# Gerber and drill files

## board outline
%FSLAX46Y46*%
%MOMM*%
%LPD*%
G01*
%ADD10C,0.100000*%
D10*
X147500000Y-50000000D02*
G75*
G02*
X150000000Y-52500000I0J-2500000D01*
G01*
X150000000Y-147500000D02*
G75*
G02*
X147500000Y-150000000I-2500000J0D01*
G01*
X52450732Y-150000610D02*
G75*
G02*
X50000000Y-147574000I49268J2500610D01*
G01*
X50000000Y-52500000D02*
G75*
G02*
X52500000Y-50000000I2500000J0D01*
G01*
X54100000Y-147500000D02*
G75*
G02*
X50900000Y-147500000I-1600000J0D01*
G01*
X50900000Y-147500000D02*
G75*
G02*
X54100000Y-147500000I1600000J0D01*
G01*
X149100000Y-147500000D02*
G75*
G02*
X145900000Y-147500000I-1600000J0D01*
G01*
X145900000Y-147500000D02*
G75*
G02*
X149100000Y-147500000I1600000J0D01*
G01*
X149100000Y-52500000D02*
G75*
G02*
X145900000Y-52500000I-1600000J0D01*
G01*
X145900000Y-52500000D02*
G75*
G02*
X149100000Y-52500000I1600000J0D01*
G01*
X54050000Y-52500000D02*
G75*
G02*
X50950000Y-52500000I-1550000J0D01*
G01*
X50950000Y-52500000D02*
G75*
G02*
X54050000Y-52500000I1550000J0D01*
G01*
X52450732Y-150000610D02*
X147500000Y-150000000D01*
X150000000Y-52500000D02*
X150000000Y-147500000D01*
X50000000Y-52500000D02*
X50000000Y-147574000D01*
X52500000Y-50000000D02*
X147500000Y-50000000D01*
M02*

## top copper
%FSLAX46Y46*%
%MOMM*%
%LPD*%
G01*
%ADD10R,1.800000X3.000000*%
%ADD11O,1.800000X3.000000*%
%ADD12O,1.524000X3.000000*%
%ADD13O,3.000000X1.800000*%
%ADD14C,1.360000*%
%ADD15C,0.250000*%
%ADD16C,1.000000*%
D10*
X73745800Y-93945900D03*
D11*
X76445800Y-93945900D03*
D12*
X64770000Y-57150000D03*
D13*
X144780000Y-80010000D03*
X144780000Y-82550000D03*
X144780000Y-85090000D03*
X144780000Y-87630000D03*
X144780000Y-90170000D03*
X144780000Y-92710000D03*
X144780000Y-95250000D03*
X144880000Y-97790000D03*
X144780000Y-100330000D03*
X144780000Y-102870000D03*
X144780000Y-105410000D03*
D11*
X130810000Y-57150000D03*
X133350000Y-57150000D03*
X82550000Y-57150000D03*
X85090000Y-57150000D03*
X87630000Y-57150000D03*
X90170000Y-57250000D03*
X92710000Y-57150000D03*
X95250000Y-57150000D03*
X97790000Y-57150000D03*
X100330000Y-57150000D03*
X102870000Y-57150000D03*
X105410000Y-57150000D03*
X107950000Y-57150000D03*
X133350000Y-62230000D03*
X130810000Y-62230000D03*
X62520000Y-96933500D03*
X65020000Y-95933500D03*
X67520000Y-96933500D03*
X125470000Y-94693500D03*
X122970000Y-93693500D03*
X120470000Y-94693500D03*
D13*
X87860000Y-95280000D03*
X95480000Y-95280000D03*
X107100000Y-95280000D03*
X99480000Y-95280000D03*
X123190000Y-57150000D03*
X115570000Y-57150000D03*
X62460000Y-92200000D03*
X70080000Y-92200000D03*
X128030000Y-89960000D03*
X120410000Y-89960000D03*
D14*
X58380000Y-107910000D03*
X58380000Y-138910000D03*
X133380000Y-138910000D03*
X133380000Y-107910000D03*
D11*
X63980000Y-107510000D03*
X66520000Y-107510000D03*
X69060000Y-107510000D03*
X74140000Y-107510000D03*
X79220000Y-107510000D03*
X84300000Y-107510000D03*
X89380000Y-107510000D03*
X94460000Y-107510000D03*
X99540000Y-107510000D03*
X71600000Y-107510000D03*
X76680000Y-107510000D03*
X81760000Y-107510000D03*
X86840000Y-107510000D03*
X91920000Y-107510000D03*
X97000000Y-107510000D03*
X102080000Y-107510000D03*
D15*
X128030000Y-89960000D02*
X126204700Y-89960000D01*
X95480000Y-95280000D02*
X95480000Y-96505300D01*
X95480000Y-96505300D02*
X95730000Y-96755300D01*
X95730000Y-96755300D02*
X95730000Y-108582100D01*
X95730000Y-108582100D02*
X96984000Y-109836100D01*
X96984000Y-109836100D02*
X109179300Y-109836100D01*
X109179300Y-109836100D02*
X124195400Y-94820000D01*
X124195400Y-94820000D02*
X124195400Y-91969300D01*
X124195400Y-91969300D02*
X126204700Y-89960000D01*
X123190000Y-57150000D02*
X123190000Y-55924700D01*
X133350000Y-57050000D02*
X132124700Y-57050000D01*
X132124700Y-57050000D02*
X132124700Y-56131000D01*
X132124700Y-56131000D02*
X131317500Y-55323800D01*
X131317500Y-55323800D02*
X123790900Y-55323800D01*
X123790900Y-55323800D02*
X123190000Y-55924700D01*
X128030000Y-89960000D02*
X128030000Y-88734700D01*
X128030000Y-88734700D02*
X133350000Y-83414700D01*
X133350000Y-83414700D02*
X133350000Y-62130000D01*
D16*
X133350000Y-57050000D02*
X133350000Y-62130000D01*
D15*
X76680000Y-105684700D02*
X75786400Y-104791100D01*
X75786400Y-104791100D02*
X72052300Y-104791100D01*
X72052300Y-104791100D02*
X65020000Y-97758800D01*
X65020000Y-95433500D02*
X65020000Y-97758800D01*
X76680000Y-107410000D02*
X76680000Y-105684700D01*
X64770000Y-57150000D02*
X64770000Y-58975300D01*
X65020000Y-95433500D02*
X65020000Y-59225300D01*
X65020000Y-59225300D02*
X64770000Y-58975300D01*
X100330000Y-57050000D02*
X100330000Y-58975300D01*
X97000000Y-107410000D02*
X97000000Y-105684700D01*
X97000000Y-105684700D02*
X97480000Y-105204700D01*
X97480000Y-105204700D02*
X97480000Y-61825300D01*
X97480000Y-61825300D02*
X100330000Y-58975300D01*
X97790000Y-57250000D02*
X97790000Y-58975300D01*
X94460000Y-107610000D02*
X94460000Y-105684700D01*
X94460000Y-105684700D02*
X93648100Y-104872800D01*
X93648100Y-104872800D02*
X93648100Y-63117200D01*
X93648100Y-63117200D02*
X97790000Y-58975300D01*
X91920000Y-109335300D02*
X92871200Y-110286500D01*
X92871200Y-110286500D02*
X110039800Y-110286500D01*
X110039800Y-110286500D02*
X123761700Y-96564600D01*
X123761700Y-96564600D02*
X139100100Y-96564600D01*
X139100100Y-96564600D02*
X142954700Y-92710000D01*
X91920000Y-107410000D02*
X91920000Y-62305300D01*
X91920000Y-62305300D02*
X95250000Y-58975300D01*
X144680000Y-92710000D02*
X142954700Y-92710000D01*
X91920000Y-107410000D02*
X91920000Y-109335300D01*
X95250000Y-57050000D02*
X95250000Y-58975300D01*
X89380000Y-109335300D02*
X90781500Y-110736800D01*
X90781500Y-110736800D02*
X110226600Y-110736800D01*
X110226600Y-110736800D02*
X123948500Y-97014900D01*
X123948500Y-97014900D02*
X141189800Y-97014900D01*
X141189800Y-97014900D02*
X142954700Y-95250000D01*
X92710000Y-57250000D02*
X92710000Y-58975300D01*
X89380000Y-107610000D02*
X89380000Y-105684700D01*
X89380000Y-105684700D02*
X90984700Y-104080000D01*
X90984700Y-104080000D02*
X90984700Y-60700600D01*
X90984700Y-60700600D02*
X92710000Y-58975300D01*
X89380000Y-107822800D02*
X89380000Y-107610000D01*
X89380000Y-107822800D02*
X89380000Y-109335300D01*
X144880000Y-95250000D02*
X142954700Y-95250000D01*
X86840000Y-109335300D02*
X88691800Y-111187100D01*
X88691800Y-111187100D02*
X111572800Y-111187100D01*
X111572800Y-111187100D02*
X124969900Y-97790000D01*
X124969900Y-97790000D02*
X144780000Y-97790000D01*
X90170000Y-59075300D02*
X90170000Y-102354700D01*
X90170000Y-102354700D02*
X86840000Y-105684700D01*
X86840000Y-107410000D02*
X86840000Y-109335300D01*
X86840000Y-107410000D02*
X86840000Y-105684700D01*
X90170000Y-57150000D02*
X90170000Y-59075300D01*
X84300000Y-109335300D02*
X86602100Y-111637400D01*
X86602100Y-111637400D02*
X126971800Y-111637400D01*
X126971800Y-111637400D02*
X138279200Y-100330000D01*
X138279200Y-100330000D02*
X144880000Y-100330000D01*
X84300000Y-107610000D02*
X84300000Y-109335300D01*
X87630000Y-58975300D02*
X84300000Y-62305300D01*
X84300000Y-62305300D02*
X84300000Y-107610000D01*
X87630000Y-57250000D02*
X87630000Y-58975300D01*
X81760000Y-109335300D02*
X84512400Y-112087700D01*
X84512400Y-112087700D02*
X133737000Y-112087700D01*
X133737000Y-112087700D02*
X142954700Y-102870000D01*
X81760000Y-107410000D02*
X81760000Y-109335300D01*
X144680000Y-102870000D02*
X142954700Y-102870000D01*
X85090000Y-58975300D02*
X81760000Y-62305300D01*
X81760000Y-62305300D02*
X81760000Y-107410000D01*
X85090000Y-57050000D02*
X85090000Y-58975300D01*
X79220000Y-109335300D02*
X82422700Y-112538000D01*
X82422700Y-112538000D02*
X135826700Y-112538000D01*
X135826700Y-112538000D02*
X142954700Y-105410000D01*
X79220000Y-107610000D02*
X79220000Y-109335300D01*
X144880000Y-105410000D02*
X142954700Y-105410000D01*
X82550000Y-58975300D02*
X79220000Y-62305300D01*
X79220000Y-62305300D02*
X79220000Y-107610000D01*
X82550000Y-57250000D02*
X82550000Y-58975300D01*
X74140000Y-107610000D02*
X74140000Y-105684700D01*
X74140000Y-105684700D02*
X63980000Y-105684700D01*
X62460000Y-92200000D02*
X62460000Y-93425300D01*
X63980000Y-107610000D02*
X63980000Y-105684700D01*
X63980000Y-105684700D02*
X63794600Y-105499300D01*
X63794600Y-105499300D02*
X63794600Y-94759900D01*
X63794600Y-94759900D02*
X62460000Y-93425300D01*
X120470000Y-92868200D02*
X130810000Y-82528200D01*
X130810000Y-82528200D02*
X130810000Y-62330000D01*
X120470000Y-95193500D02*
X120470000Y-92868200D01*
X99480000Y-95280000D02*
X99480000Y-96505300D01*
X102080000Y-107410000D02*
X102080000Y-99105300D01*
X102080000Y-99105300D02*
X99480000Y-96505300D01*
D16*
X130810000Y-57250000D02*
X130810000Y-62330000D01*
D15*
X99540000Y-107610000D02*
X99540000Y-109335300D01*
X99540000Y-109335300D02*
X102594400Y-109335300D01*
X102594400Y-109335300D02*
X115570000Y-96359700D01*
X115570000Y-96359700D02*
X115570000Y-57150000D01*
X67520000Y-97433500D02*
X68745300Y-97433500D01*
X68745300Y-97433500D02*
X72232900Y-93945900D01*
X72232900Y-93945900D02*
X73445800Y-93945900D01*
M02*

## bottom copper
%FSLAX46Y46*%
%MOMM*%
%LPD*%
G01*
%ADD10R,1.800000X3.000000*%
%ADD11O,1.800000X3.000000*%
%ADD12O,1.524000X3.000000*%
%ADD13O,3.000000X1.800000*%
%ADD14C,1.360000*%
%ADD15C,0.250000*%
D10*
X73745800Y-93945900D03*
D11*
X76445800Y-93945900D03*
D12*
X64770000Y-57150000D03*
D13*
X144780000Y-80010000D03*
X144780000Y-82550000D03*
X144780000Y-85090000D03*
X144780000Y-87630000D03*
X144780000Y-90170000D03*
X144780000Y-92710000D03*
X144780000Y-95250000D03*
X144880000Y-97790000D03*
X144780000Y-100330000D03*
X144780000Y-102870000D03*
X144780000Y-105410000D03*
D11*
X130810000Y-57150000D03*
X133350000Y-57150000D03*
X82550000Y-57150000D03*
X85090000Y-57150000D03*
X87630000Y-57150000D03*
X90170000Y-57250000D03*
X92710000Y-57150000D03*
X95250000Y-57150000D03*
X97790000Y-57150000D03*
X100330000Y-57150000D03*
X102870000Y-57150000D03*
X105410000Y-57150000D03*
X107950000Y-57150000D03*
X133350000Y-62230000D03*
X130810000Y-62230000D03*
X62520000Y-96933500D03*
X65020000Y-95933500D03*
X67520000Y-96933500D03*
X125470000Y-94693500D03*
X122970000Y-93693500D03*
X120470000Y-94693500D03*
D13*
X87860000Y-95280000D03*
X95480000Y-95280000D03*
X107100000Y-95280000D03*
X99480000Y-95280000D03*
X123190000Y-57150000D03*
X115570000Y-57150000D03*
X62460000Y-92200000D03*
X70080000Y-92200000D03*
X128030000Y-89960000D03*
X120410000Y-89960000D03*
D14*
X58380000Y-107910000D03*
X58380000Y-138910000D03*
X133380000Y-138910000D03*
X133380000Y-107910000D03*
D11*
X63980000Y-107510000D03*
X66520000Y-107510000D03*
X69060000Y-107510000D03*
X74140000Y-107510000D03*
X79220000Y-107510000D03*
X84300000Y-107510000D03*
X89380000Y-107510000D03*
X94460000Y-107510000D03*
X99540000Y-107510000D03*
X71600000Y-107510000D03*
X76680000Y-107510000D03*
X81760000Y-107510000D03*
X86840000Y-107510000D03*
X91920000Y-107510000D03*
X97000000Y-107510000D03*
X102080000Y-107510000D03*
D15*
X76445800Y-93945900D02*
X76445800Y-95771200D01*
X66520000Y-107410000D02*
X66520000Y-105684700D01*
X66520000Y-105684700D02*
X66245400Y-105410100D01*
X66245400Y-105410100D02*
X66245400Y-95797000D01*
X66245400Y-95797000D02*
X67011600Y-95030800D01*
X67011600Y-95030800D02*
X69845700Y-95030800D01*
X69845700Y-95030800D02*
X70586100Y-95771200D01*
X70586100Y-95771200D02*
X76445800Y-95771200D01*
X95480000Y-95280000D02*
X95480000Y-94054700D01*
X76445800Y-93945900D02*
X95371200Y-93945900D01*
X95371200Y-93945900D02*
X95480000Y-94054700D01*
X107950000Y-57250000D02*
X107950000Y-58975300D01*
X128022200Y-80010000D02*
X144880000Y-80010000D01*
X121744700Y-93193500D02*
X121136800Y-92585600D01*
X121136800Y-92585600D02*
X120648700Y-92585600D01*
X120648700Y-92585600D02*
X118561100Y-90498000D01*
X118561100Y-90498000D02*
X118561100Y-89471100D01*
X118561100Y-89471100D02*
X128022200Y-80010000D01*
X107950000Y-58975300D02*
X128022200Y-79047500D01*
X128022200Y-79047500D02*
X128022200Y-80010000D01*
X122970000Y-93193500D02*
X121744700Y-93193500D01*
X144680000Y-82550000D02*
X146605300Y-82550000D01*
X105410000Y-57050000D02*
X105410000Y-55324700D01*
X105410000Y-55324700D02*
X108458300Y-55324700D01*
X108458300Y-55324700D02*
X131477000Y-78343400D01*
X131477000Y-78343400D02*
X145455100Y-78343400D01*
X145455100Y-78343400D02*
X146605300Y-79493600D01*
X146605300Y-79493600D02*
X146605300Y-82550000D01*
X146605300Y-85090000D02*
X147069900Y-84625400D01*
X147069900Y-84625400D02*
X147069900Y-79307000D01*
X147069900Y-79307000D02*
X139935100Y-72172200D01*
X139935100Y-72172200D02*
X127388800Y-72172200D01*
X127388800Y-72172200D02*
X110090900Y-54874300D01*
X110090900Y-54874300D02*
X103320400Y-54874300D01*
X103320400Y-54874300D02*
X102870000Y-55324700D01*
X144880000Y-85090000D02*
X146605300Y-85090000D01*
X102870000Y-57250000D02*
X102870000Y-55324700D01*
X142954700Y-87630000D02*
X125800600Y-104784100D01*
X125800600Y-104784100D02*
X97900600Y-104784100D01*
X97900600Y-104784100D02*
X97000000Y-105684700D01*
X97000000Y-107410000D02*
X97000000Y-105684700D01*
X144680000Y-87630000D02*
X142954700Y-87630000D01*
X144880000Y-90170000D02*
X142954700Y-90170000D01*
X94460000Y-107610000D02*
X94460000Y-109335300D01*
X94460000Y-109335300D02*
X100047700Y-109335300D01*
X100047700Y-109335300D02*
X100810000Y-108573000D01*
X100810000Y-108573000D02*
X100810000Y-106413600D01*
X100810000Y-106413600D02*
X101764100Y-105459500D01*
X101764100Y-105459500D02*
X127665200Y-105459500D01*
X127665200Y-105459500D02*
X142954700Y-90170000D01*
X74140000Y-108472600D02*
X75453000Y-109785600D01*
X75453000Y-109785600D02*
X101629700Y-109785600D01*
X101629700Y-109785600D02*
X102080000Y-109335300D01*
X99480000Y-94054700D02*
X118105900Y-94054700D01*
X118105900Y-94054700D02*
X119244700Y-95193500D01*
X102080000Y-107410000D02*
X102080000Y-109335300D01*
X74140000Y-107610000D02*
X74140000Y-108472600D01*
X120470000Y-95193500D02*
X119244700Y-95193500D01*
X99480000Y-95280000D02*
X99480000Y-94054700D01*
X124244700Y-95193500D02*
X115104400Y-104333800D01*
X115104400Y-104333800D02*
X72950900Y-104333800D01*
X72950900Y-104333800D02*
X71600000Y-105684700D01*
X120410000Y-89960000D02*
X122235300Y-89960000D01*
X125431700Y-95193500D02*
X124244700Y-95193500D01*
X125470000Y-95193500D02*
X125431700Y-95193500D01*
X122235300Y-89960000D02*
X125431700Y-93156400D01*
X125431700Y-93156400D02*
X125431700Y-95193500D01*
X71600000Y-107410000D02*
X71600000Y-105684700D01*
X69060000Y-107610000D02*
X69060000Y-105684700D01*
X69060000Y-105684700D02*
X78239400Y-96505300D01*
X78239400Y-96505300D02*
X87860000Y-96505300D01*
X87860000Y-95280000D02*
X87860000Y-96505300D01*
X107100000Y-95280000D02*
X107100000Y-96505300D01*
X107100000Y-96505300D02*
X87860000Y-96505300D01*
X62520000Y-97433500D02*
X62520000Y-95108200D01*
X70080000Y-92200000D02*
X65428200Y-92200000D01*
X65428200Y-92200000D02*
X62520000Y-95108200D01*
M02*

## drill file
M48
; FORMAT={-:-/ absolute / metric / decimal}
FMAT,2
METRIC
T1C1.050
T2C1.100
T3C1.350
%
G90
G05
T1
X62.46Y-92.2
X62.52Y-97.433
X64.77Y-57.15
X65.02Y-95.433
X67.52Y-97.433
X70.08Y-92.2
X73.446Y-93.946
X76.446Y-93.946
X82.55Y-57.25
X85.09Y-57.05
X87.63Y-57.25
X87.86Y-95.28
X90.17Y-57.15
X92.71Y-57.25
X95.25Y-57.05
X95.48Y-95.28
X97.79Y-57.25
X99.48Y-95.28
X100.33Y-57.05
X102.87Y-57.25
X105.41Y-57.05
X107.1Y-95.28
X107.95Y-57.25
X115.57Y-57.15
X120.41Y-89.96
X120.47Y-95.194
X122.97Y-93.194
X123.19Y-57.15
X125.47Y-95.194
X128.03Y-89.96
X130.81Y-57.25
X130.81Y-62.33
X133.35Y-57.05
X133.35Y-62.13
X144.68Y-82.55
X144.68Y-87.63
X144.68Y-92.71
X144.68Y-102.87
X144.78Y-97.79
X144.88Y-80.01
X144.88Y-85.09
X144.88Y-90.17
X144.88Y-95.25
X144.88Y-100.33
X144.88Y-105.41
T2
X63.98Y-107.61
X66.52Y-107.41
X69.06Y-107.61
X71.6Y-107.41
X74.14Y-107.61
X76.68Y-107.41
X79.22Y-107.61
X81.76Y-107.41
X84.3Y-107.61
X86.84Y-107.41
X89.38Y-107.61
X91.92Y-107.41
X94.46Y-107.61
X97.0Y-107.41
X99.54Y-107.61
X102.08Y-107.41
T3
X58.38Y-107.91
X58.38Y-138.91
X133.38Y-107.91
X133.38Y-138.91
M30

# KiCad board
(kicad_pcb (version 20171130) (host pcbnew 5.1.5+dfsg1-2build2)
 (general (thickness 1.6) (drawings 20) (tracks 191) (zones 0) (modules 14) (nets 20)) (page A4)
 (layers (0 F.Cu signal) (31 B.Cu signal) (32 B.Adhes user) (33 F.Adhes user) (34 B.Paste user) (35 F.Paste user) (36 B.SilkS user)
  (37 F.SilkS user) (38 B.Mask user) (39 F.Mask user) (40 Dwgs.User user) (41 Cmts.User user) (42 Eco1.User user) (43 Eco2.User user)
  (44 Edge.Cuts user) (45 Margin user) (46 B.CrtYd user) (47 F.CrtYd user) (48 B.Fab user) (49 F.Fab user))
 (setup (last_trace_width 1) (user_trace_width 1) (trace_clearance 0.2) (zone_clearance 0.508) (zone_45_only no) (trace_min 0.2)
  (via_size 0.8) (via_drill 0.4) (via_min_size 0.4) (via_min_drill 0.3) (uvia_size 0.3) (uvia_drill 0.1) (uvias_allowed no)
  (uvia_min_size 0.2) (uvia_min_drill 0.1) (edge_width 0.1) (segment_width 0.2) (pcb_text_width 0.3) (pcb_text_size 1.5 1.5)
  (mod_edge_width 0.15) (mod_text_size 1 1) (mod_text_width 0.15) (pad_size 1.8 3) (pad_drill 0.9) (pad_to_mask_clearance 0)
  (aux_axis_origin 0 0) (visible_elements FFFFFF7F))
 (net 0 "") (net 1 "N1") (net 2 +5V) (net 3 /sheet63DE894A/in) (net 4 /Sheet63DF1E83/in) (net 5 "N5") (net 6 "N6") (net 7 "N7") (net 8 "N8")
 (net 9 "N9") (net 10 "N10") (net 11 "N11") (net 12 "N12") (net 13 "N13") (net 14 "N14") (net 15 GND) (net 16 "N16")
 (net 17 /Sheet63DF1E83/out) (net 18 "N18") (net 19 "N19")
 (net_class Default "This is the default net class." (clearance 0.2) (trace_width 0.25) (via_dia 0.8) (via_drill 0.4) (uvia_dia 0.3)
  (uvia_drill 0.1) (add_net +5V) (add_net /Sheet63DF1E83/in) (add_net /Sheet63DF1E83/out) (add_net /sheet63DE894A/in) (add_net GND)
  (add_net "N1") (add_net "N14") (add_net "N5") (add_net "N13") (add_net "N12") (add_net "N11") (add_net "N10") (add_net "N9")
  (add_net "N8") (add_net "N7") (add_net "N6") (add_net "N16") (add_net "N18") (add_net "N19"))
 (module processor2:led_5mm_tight (layer F.Cu) (at 74.9458 93.9459)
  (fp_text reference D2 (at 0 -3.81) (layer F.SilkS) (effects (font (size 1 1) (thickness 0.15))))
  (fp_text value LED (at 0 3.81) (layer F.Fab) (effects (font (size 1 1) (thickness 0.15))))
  (pad 1 thru_hole rect (at -1.5 0) (size 1.8 3) (drill 1.05 (offset 0.3 0)) (layers *.Cu *.Mask) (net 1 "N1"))
  (pad 2 thru_hole oval (at 1.5 0) (size 1.8 3) (drill 1.05) (layers *.Cu *.Mask) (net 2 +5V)))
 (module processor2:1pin (layer F.Cu) (at 64.77 57.15 90)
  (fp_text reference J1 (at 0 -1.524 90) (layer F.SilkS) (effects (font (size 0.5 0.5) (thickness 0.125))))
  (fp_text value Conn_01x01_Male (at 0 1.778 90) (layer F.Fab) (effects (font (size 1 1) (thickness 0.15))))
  (pad 1 thru_hole oval (at 0 0 90) (size 3 1.524) (drill 1.05) (layers *.Cu *.Mask) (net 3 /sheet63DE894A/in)))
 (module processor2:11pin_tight (layer F.Cu) (at 144.78 105.41 90)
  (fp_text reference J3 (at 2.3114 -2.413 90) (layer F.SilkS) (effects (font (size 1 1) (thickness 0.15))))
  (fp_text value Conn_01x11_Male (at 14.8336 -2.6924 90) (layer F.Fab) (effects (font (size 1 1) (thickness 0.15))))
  (pad 11 thru_hole oval (at 25.4 0.1 90) (size 1.8 3) (drill 1.05 (offset 0 -0.1)) (layers *.Cu *.Mask) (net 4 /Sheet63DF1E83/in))
  (pad 10 thru_hole oval (at 22.86 -0.1 90) (size 1.8 3) (drill 1.05 (offset 0 0.1)) (layers *.Cu *.Mask) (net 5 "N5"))
  (pad 9 thru_hole oval (at 20.32 0.1 90) (size 1.8 3) (drill 1.05 (offset 0 -0.1)) (layers *.Cu *.Mask) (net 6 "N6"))
  (pad 8 thru_hole oval (at 17.78 -0.1 90) (size 1.8 3) (drill 1.05 (offset 0 0.1)) (layers *.Cu *.Mask) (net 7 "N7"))
  (pad 7 thru_hole oval (at 15.24 0.1 90) (size 1.8 3) (drill 1.05 (offset 0 -0.1)) (layers *.Cu *.Mask) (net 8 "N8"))
  (pad 6 thru_hole oval (at 12.7 -0.1 90) (size 1.8 3) (drill 1.05 (offset 0 0.1)) (layers *.Cu *.Mask) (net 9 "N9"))
  (pad 5 thru_hole oval (at 10.16 0.1 90) (size 1.8 3) (drill 1.05 (offset 0 -0.1)) (layers *.Cu *.Mask) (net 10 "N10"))
  (pad 4 thru_hole oval (at 7.62 0 90) (size 1.8 3) (drill 1.05 (offset 0 0.1)) (layers *.Cu *.Mask) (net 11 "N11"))
  (pad 3 thru_hole oval (at 5.08 0.1 90) (size 1.8 3) (drill 1.05 (offset 0 -0.1)) (layers *.Cu *.Mask) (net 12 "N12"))
  (pad 2 thru_hole oval (at 2.54 -0.1 90) (size 1.8 3) (drill 1.05 (offset 0 0.1)) (layers *.Cu *.Mask) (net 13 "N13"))
  (pad 1 thru_hole oval (at 0 0.1 90) (size 1.8 3) (drill 1.05 (offset 0 -0.1)) (layers *.Cu *.Mask) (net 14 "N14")))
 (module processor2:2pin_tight (layer F.Cu) (at 133.35 57.15)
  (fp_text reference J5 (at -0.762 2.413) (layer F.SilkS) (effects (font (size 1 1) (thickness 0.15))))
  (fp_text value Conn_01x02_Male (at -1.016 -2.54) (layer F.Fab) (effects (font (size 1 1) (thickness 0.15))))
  (pad 2 thru_hole oval (at -2.54 0.1) (size 1.8 3) (drill 1.05 (offset 0 -0.1)) (layers *.Cu *.Mask) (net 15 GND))
  (pad 1 thru_hole oval (at 0 -0.1) (size 1.8 3) (drill 1.05 (offset 0 0.1)) (layers *.Cu *.Mask) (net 2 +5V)))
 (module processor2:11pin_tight (layer F.Cu) (at 82.55 57.15)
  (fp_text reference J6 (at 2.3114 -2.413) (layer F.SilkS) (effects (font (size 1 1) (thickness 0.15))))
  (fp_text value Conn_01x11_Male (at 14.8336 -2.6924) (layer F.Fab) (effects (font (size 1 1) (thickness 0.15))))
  (pad 1 thru_hole oval (at 0 0.1) (size 1.8 3) (drill 1.05 (offset 0 -0.1)) (layers *.Cu *.Mask) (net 14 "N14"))
  (pad 2 thru_hole oval (at 2.54 -0.1) (size 1.8 3) (drill 1.05 (offset 0 0.1)) (layers *.Cu *.Mask) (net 13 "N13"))
  (pad 3 thru_hole oval (at 5.08 0.1) (size 1.8 3) (drill 1.05 (offset 0 -0.1)) (layers *.Cu *.Mask) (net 12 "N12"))
  (pad 4 thru_hole oval (at 7.62 0) (size 1.8 3) (drill 1.05 (offset 0 0.1)) (layers *.Cu *.Mask) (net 11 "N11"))
  (pad 5 thru_hole oval (at 10.16 0.1) (size 1.8 3) (drill 1.05 (offset 0 -0.1)) (layers *.Cu *.Mask) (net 10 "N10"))
  (pad 6 thru_hole oval (at 12.7 -0.1) (size 1.8 3) (drill 1.05 (offset 0 0.1)) (layers *.Cu *.Mask) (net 9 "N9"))
  (pad 7 thru_hole oval (at 15.24 0.1) (size 1.8 3) (drill 1.05 (offset 0 -0.1)) (layers *.Cu *.Mask) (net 8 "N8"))
  (pad 8 thru_hole oval (at 17.78 -0.1) (size 1.8 3) (drill 1.05 (offset 0 0.1)) (layers *.Cu *.Mask) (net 7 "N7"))
  (pad 9 thru_hole oval (at 20.32 0.1) (size 1.8 3) (drill 1.05 (offset 0 -0.1)) (layers *.Cu *.Mask) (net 6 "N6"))
  (pad 10 thru_hole oval (at 22.86 -0.1) (size 1.8 3) (drill 1.05 (offset 0 0.1)) (layers *.Cu *.Mask) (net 5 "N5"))
  (pad 11 thru_hole oval (at 25.4 0.1) (size 1.8 3) (drill 1.05 (offset 0 -0.1)) (layers *.Cu *.Mask) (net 4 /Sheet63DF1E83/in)))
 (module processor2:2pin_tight (layer F.Cu) (at 133.35 62.23)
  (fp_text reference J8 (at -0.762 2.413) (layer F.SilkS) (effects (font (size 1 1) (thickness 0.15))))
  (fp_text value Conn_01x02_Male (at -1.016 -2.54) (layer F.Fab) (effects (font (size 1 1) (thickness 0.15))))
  (pad 1 thru_hole oval (at 0 -0.1) (size 1.8 3) (drill 1.05 (offset 0 0.1)) (layers *.Cu *.Mask) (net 2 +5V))
  (pad 2 thru_hole oval (at -2.54 0.1) (size 1.8 3) (drill 1.05 (offset 0 -0.1)) (layers *.Cu *.Mask) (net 15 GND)))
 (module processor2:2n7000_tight (layer F.Cu) (at 65.02 96.4335)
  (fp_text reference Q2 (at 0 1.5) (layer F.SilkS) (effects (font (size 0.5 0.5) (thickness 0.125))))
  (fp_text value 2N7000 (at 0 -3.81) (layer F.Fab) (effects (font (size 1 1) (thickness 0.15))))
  (pad 1 thru_hole oval (at -2.5 1) (size 1.8 3) (drill 1.05 (offset 0 -0.5)) (layers *.Cu *.Mask) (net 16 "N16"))
  (pad 2 thru_hole oval (at 0 -1) (size 1.8 3) (drill 1.05 (offset 0 0.5)) (layers *.Cu *.Mask) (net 3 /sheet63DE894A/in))
  (pad 3 thru_hole oval (at 2.5 1) (size 1.8 3) (drill 1.05 (offset 0 -0.5)) (layers *.Cu *.Mask) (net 1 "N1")))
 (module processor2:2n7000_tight (layer F.Cu) (at 122.97 94.1935)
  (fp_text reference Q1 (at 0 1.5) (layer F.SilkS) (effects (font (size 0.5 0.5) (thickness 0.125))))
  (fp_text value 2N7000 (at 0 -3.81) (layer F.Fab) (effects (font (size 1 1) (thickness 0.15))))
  (pad 3 thru_hole oval (at 2.5 1) (size 1.8 3) (drill 1.05 (offset 0 -0.5)) (layers *.Cu *.Mask) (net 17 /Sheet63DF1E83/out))
  (pad 2 thru_hole oval (at 0 -1) (size 1.8 3) (drill 1.05 (offset 0 0.5)) (layers *.Cu *.Mask) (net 4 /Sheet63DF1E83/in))
  (pad 1 thru_hole oval (at -2.5 1) (size 1.8 3) (drill 1.05 (offset 0 -0.5)) (layers *.Cu *.Mask) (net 15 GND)))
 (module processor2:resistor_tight (layer F.Cu) (at 91.67 95.28)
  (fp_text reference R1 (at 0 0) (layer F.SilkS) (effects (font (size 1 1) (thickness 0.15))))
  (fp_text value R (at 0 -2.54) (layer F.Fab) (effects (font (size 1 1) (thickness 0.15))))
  (pad 2 thru_hole oval (at -3.81 0 90) (size 1.8 3) (drill 1.05) (layers *.Cu *.Mask) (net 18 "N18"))
  (pad 1 thru_hole oval (at 3.81 0 90) (size 1.8 3) (drill 1.05) (layers *.Cu *.Mask) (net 2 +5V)))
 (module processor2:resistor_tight (layer F.Cu) (at 103.29 95.28)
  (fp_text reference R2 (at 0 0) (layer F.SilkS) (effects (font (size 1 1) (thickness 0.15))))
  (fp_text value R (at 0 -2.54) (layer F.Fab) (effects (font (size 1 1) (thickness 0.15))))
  (pad 1 thru_hole oval (at 3.81 0 90) (size 1.8 3) (drill 1.05) (layers *.Cu *.Mask) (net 18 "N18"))
  (pad 2 thru_hole oval (at -3.81 0 90) (size 1.8 3) (drill 1.05) (layers *.Cu *.Mask) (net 15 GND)))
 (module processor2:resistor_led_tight (layer F.Cu) (at 119.38 57.15)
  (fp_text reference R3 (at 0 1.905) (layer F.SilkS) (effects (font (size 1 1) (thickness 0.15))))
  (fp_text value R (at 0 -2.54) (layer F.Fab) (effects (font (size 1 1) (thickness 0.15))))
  (pad 1 thru_hole oval (at 3.81 0 90) (size 1.8 3) (drill 1.05) (layers *.Cu *.Mask) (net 2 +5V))
  (pad 2 thru_hole oval (at -3.81 0 90) (size 1.8 3) (drill 1.05) (layers *.Cu *.Mask) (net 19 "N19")))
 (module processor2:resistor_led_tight (layer F.Cu) (at 66.27 92.2)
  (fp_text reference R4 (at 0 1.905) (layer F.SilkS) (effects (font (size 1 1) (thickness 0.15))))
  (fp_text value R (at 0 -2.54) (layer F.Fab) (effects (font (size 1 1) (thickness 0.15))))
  (pad 2 thru_hole oval (at -3.81 0 90) (size 1.8 3) (drill 1.05) (layers *.Cu *.Mask) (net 15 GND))
  (pad 1 thru_hole oval (at 3.81 0 90) (size 1.8 3) (drill 1.05) (layers *.Cu *.Mask) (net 16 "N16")))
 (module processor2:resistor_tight (layer F.Cu) (at 124.22 89.96)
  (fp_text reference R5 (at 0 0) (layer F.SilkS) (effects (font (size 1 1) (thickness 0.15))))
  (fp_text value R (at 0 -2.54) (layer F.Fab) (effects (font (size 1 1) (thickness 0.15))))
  (pad 1 thru_hole oval (at 3.81 0 90) (size 1.8 3) (drill 1.05) (layers *.Cu *.Mask) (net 2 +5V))
  (pad 2 thru_hole oval (at -3.81 0 90) (size 1.8 3) (drill 1.05) (layers *.Cu *.Mask) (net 17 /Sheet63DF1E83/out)))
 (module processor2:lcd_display (layer F.Cu) (at 55.88 105.41)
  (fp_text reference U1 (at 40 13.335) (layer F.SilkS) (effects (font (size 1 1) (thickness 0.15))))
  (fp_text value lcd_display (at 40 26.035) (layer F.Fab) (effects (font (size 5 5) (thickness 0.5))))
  (pad "" np_thru_hole circle (at 2.5 2.5) (size 1.36 1.36) (drill 1.35) (layers *.Cu *.Mask))
  (pad "" np_thru_hole circle (at 2.5 33.5) (size 1.36 1.36) (drill 1.35) (layers *.Cu *.Mask))
  (pad "" np_thru_hole circle (at 77.5 33.5) (size 1.36 1.36) (drill 1.35) (layers *.Cu *.Mask))
  (pad "" np_thru_hole circle (at 77.5 2.5) (size 1.36 1.36) (drill 1.35) (layers *.Cu *.Mask))
  (pad gnd thru_hole oval (at 8.1 2.2) (size 1.8 3) (drill 1.1 (offset 0 -0.1)) (layers *.Cu *.Mask) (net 15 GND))
  (pad 5v thru_hole oval (at 10.64 2) (size 1.8 3) (drill 1.1 (offset 0 0.1)) (layers *.Cu *.Mask) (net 2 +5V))
  (pad contrast thru_hole oval (at 13.18 2.2) (size 1.8 3) (drill 1.1 (offset 0 -0.1)) (layers *.Cu *.Mask) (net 18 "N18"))
  (pad read/write thru_hole oval (at 18.26 2.2) (size 1.8 3) (drill 1.1 (offset 0 -0.1)) (layers *.Cu *.Mask) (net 15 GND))
  (pad d0 thru_hole oval (at 23.34 2.2) (size 1.8 3) (drill 1.1 (offset 0 -0.1)) (layers *.Cu *.Mask) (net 14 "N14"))
  (pad d2 thru_hole oval (at 28.42 2.2) (size 1.8 3) (drill 1.1 (offset 0 -0.1)) (layers *.Cu *.Mask) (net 12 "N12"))
  (pad d4 thru_hole oval (at 33.5 2.2) (size 1.8 3) (drill 1.1 (offset 0 -0.1)) (layers *.Cu *.Mask) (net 10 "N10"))
  (pad d6 thru_hole oval (at 38.58 2.2) (size 1.8 3) (drill 1.1 (offset 0 -0.1)) (layers *.Cu *.Mask) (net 8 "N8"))
  (pad led_positive thru_hole oval (at 43.66 2.2) (size 1.8 3) (drill 1.1 (offset 0 -0.1)) (layers *.Cu *.Mask) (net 19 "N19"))
  (pad register_select thru_hole oval (at 15.72 2) (size 1.8 3) (drill 1.1 (offset 0 0.1)) (layers *.Cu *.Mask) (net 17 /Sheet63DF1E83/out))
  (pad enable thru_hole oval (at 20.8 2) (size 1.8 3) (drill 1.1 (offset 0 0.1)) (layers *.Cu *.Mask) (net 3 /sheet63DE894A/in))
  (pad d1 thru_hole oval (at 25.88 2) (size 1.8 3) (drill 1.1 (offset 0 0.1)) (layers *.Cu *.Mask) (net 13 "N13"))
  (pad d3 thru_hole oval (at 30.96 2) (size 1.8 3) (drill 1.1 (offset 0 0.1)) (layers *.Cu *.Mask) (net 11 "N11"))
  (pad d5 thru_hole oval (at 36.04 2) (size 1.8 3) (drill 1.1 (offset 0 0.1)) (layers *.Cu *.Mask) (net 9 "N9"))
  (pad d7 thru_hole oval (at 41.12 2) (size 1.8 3) (drill 1.1 (offset 0 0.1)) (layers *.Cu *.Mask) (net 7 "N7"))
  (pad led_negative thru_hole oval (at 46.2 2) (size 1.8 3) (drill 1.1 (offset 0 0.1)) (layers *.Cu *.Mask) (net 15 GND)))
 (gr_arc (start 147.5 52.5) (end 147.5 50) (angle 90) (layer Edge.Cuts) (width 0.1))
 (gr_arc (start 147.5 147.5) (end 150 147.5) (angle 90) (layer Edge.Cuts) (width 0.1))
 (gr_arc (start 52.5 147.5) (end 50 147.574) (angle -87.17581862) (layer Edge.Cuts) (width 0.1))
 (gr_arc (start 52.5 52.5) (end 52.5 50) (angle -90) (layer Edge.Cuts) (width 0.1))
 (gr_circle (center 52.5 147.5) (end 54.1 147.5) (layer Edge.Cuts) (width 0.1))
 (gr_circle (center 147.5 147.5) (end 149.1 147.5) (layer Edge.Cuts) (width 0.1))
 (gr_circle (center 147.5 52.5) (end 149.1 52.5) (layer Edge.Cuts) (width 0.1))
 (gr_circle (center 52.5 52.5) (end 54.05 52.5) (layer Edge.Cuts) (width 0.1))
 (gr_line (start 52.450732 150.00061) (end 147.5 150) (layer Edge.Cuts) (width 0.1))
 (gr_line (start 150 52.5) (end 150 147.5) (layer Edge.Cuts) (width 0.1))
 (gr_line (start 50 52.5) (end 50 147.574) (layer Edge.Cuts) (width 0.1))
 (gr_line (start 52.5 50) (end 147.5 50) (layer Edge.Cuts) (width 0.1))
 (segment (start 128.03 89.96) (end 126.2047 89.96) (width 0.25) (layer F.Cu) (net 2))
 (segment (start 95.48 95.28) (end 95.48 96.5053) (width 0.25) (layer F.Cu) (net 2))
 (segment (start 95.48 96.5053) (end 95.73 96.7553) (width 0.25) (layer F.Cu) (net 2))
 (segment (start 95.73 96.7553) (end 95.73 108.5821) (width 0.25) (layer F.Cu) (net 2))
 (segment (start 95.73 108.5821) (end 96.984 109.8361) (width 0.25) (layer F.Cu) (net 2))
 (segment (start 96.984 109.8361) (end 109.1793 109.8361) (width 0.25) (layer F.Cu) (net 2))
 (segment (start 109.1793 109.8361) (end 124.1954 94.82) (width 0.25) (layer F.Cu) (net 2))
 (segment (start 124.1954 94.82) (end 124.1954 91.9693) (width 0.25) (layer F.Cu) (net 2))
 (segment (start 124.1954 91.9693) (end 126.2047 89.96) (width 0.25) (layer F.Cu) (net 2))
 (segment (start 76.4458 93.9459) (end 76.4458 95.7712) (width 0.25) (layer B.Cu) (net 2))
 (segment (start 66.52 107.41) (end 66.52 105.6847) (width 0.25) (layer B.Cu) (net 2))
 (segment (start 66.52 105.6847) (end 66.2454 105.4101) (width 0.25) (layer B.Cu) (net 2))
 (segment (start 66.2454 105.4101) (end 66.2454 95.797) (width 0.25) (layer B.Cu) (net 2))
 (segment (start 66.2454 95.797) (end 67.0116 95.0308) (width 0.25) (layer B.Cu) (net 2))
 (segment (start 67.0116 95.0308) (end 69.8457 95.0308) (width 0.25) (layer B.Cu) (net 2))
 (segment (start 69.8457 95.0308) (end 70.5861 95.7712) (width 0.25) (layer B.Cu) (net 2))
 (segment (start 70.5861 95.7712) (end 76.4458 95.7712) (width 0.25) (layer B.Cu) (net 2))
 (segment (start 123.19 57.15) (end 123.19 55.9247) (width 0.25) (layer F.Cu) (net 2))
 (segment (start 133.35 57.05) (end 132.1247 57.05) (width 0.25) (layer F.Cu) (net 2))
 (segment (start 132.1247 57.05) (end 132.1247 56.131) (width 0.25) (layer F.Cu) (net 2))
 (segment (start 132.1247 56.131) (end 131.3175 55.3238) (width 0.25) (layer F.Cu) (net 2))
 (segment (start 131.3175 55.3238) (end 123.7909 55.3238) (width 0.25) (layer F.Cu) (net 2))
 (segment (start 123.7909 55.3238) (end 123.19 55.9247) (width 0.25) (layer F.Cu) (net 2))
 (segment (start 128.03 89.96) (end 128.03 88.7347) (width 0.25) (layer F.Cu) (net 2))
 (segment (start 128.03 88.7347) (end 133.35 83.4147) (width 0.25) (layer F.Cu) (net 2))
 (segment (start 133.35 83.4147) (end 133.35 62.13) (width 0.25) (layer F.Cu) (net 2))
 (segment (start 95.48 95.28) (end 95.48 94.0547) (width 0.25) (layer B.Cu) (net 2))
 (segment (start 76.4458 93.9459) (end 95.3712 93.9459) (width 0.25) (layer B.Cu) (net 2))
 (segment (start 95.3712 93.9459) (end 95.48 94.0547) (width 0.25) (layer B.Cu) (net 2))
 (segment (start 133.35 57.05) (end 133.35 62.13) (width 1) (layer F.Cu) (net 2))
 (segment (start 76.68 105.6847) (end 75.7864 104.7911) (width 0.25) (layer F.Cu) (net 3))
 (segment (start 75.7864 104.7911) (end 72.0523 104.7911) (width 0.25) (layer F.Cu) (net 3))
 (segment (start 72.0523 104.7911) (end 65.02 97.7588) (width 0.25) (layer F.Cu) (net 3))
 (segment (start 65.02 95.4335) (end 65.02 97.7588) (width 0.25) (layer F.Cu) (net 3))
 (segment (start 76.68 107.41) (end 76.68 105.6847) (width 0.25) (layer F.Cu) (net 3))
 (segment (start 64.77 57.15) (end 64.77 58.9753) (width 0.25) (layer F.Cu) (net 3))
 (segment (start 65.02 95.4335) (end 65.02 59.2253) (width 0.25) (layer F.Cu) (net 3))
 (segment (start 65.02 59.2253) (end 64.77 58.9753) (width 0.25) (layer F.Cu) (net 3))
 (segment (start 107.95 57.25) (end 107.95 58.9753) (width 0.25) (layer B.Cu) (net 4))
 (segment (start 128.0222 80.01) (end 144.88 80.01) (width 0.25) (layer B.Cu) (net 4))
 (segment (start 121.7447 93.1935) (end 121.1368 92.5856) (width 0.25) (layer B.Cu) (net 4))
 (segment (start 121.1368 92.5856) (end 120.6487 92.5856) (width 0.25) (layer B.Cu) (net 4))
 (segment (start 120.6487 92.5856) (end 118.5611 90.498) (width 0.25) (layer B.Cu) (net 4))
 (segment (start 118.5611 90.498) (end 118.5611 89.4711) (width 0.25) (layer B.Cu) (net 4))
 (segment (start 118.5611 89.4711) (end 128.0222 80.01) (width 0.25) (layer B.Cu) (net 4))
 (segment (start 107.95 58.9753) (end 128.0222 79.0475) (width 0.25) (layer B.Cu) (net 4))
 (segment (start 128.0222 79.0475) (end 128.0222 80.01) (width 0.25) (layer B.Cu) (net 4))
 (segment (start 122.97 93.1935) (end 121.7447 93.1935) (width 0.25) (layer B.Cu) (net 4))
 (segment (start 144.68 82.55) (end 146.6053 82.55) (width 0.25) (layer B.Cu) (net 5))
 (segment (start 105.41 57.05) (end 105.41 55.3247) (width 0.25) (layer B.Cu) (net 5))
 (segment (start 105.41 55.3247) (end 108.4583 55.3247) (width 0.25) (layer B.Cu) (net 5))
 (segment (start 108.4583 55.3247) (end 131.477 78.3434) (width 0.25) (layer B.Cu) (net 5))
 (segment (start 131.477 78.3434) (end 145.4551 78.3434) (width 0.25) (layer B.Cu) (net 5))
 (segment (start 145.4551 78.3434) (end 146.6053 79.4936) (width 0.25) (layer B.Cu) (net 5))
 (segment (start 146.6053 79.4936) (end 146.6053 82.55) (width 0.25) (layer B.Cu) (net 5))
 (segment (start 146.6053 85.09) (end 147.0699 84.6254) (width 0.25) (layer B.Cu) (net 6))
 (segment (start 147.0699 84.6254) (end 147.0699 79.307) (width 0.25) (layer B.Cu) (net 6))
 (segment (start 147.0699 79.307) (end 139.9351 72.1722) (width 0.25) (layer B.Cu) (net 6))
 (segment (start 139.9351 72.1722) (end 127.3888 72.1722) (width 0.25) (layer B.Cu) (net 6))
 (segment (start 127.3888 72.1722) (end 110.0909 54.8743) (width 0.25) (layer B.Cu) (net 6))
 (segment (start 110.0909 54.8743) (end 103.3204 54.8743) (width 0.25) (layer B.Cu) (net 6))
 (segment (start 103.3204 54.8743) (end 102.87 55.3247) (width 0.25) (layer B.Cu) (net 6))
 (segment (start 144.88 85.09) (end 146.6053 85.09) (width 0.25) (layer B.Cu) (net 6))
 (segment (start 102.87 57.25) (end 102.87 55.3247) (width 0.25) (layer B.Cu) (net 6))
 (segment (start 142.9547 87.63) (end 125.8006 104.7841) (width 0.25) (layer B.Cu) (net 7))
 (segment (start 125.8006 104.7841) (end 97.9006 104.7841) (width 0.25) (layer B.Cu) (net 7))
 (segment (start 97.9006 104.7841) (end 97 105.6847) (width 0.25) (layer B.Cu) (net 7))
 (segment (start 97 107.41) (end 97 105.6847) (width 0.25) (layer B.Cu) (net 7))
 (segment (start 144.68 87.63) (end 142.9547 87.63) (width 0.25) (layer B.Cu) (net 7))
 (segment (start 100.33 57.05) (end 100.33 58.9753) (width 0.25) (layer F.Cu) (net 7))
 (segment (start 97 107.41) (end 97 105.6847) (width 0.25) (layer F.Cu) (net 7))
 (segment (start 97 105.6847) (end 97.48 105.2047) (width 0.25) (layer F.Cu) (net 7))
 (segment (start 97.48 105.2047) (end 97.48 61.8253) (width 0.25) (layer F.Cu) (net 7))
 (segment (start 97.48 61.8253) (end 100.33 58.9753) (width 0.25) (layer F.Cu) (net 7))
 (segment (start 144.88 90.17) (end 142.9547 90.17) (width 0.25) (layer B.Cu) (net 8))
 (segment (start 94.46 107.61) (end 94.46 109.3353) (width 0.25) (layer B.Cu) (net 8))
 (segment (start 94.46 109.3353) (end 100.0477 109.3353) (width 0.25) (layer B.Cu) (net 8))
 (segment (start 100.0477 109.3353) (end 100.81 108.573) (width 0.25) (layer B.Cu) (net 8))
 (segment (start 100.81 108.573) (end 100.81 106.4136) (width 0.25) (layer B.Cu) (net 8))
 (segment (start 100.81 106.4136) (end 101.7641 105.4595) (width 0.25) (layer B.Cu) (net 8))
 (segment (start 101.7641 105.4595) (end 127.6652 105.4595) (width 0.25) (layer B.Cu) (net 8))
 (segment (start 127.6652 105.4595) (end 142.9547 90.17) (width 0.25) (layer B.Cu) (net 8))
 (segment (start 97.79 57.25) (end 97.79 58.9753) (width 0.25) (layer F.Cu) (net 8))
 (segment (start 94.46 107.61) (end 94.46 105.6847) (width 0.25) (layer F.Cu) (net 8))
 (segment (start 94.46 105.6847) (end 93.6481 104.8728) (width 0.25) (layer F.Cu) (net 8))
 (segment (start 93.6481 104.8728) (end 93.6481 63.1172) (width 0.25) (layer F.Cu) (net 8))
 (segment (start 93.6481 63.1172) (end 97.79 58.9753) (width 0.25) (layer F.Cu) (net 8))
 (segment (start 91.92 109.3353) (end 92.8712 110.2865) (width 0.25) (layer F.Cu) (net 9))
 (segment (start 92.8712 110.2865) (end 110.0398 110.2865) (width 0.25) (layer F.Cu) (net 9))
 (segment (start 110.0398 110.2865) (end 123.7617 96.5646) (width 0.25) (layer F.Cu) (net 9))
 (segment (start 123.7617 96.5646) (end 139.1001 96.5646) (width 0.25) (layer F.Cu) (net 9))
 (segment (start 139.1001 96.5646) (end 142.9547 92.71) (width 0.25) (layer F.Cu) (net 9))
 (segment (start 91.92 107.41) (end 91.92 62.3053) (width 0.25) (layer F.Cu) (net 9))
 (segment (start 91.92 62.3053) (end 95.25 58.9753) (width 0.25) (layer F.Cu) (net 9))
 (segment (start 144.68 92.71) (end 142.9547 92.71) (width 0.25) (layer F.Cu) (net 9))
 (segment (start 91.92 107.41) (end 91.92 109.3353) (width 0.25) (layer F.Cu) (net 9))
 (segment (start 95.25 57.05) (end 95.25 58.9753) (width 0.25) (layer F.Cu) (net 9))
 (segment (start 89.38 109.3353) (end 90.7815 110.7368) (width 0.25) (layer F.Cu) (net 10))
 (segment (start 90.7815 110.7368) (end 110.2266 110.7368) (width 0.25) (layer F.Cu) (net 10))
 (segment (start 110.2266 110.7368) (end 123.9485 97.0149) (width 0.25) (layer F.Cu) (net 10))
 (segment (start 123.9485 97.0149) (end 141.1898 97.0149) (width 0.25) (layer F.Cu) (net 10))
 (segment (start 141.1898 97.0149) (end 142.9547 95.25) (width 0.25) (layer F.Cu) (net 10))
 (segment (start 92.71 57.25) (end 92.71 58.9753) (width 0.25) (layer F.Cu) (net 10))
 (segment (start 89.38 107.61) (end 89.38 105.6847) (width 0.25) (layer F.Cu) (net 10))
 (segment (start 89.38 105.6847) (end 90.9847 104.08) (width 0.25) (layer F.Cu) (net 10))
 (segment (start 90.9847 104.08) (end 90.9847 60.7006) (width 0.25) (layer F.Cu) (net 10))
 (segment (start 90.9847 60.7006) (end 92.71 58.9753) (width 0.25) (layer F.Cu) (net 10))
 (segment (start 89.38 107.8228) (end 89.38 107.61) (width 0.25) (layer F.Cu) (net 10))
 (segment (start 89.38 107.8228) (end 89.38 109.3353) (width 0.25) (layer F.Cu) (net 10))
 (segment (start 144.88 95.25) (end 142.9547 95.25) (width 0.25) (layer F.Cu) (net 10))
 (segment (start 86.84 109.3353) (end 88.6918 111.1871) (width 0.25) (layer F.Cu) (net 11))
 (segment (start 88.6918 111.1871) (end 111.5728 111.1871) (width 0.25) (layer F.Cu) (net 11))
 (segment (start 111.5728 111.1871) (end 124.9699 97.79) (width 0.25) (layer F.Cu) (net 11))
 (segment (start 124.9699 97.79) (end 144.78 97.79) (width 0.25) (layer F.Cu) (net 11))
 (segment (start 90.17 59.0753) (end 90.17 102.3547) (width 0.25) (layer F.Cu) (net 11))
 (segment (start 90.17 102.3547) (end 86.84 105.6847) (width 0.25) (layer F.Cu) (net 11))
 (segment (start 86.84 107.41) (end 86.84 109.3353) (width 0.25) (layer F.Cu) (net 11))
 (segment (start 86.84 107.41) (end 86.84 105.6847) (width 0.25) (layer F.Cu) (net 11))
 (segment (start 90.17 57.15) (end 90.17 59.0753) (width 0.25) (layer F.Cu) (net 11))
 (segment (start 84.3 109.3353) (end 86.6021 111.6374) (width 0.25) (layer F.Cu) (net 12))
 (segment (start 86.6021 111.6374) (end 126.9718 111.6374) (width 0.25) (layer F.Cu) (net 12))
 (segment (start 126.9718 111.6374) (end 138.2792 100.33) (width 0.25) (layer F.Cu) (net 12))
 (segment (start 138.2792 100.33) (end 144.88 100.33) (width 0.25) (layer F.Cu) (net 12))
 (segment (start 84.3 107.61) (end 84.3 109.3353) (width 0.25) (layer F.Cu) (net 12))
 (segment (start 87.63 58.9753) (end 84.3 62.3053) (width 0.25) (layer F.Cu) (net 12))
 (segment (start 84.3 62.3053) (end 84.3 107.61) (width 0.25) (layer F.Cu) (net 12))
 (segment (start 87.63 57.25) (end 87.63 58.9753) (width 0.25) (layer F.Cu) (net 12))
 (segment (start 81.76 109.3353) (end 84.5124 112.0877) (width 0.25) (layer F.Cu) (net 13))
 (segment (start 84.5124 112.0877) (end 133.737 112.0877) (width 0.25) (layer F.Cu) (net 13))
 (segment (start 133.737 112.0877) (end 142.9547 102.87) (width 0.25) (layer F.Cu) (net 13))
 (segment (start 81.76 107.41) (end 81.76 109.3353) (width 0.25) (layer F.Cu) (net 13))
 (segment (start 144.68 102.87) (end 142.9547 102.87) (width 0.25) (layer F.Cu) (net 13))
 (segment (start 85.09 58.9753) (end 81.76 62.3053) (width 0.25) (layer F.Cu) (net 13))
 (segment (start 81.76 62.3053) (end 81.76 107.41) (width 0.25) (layer F.Cu) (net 13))
 (segment (start 85.09 57.05) (end 85.09 58.9753) (width 0.25) (layer F.Cu) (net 13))
 (segment (start 79.22 109.3353) (end 82.4227 112.538) (width 0.25) (layer F.Cu) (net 14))
 (segment (start 82.4227 112.538) (end 135.8267 112.538) (width 0.25) (layer F.Cu) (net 14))
 (segment (start 135.8267 112.538) (end 142.9547 105.41) (width 0.25) (layer F.Cu) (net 14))
 (segment (start 79.22 107.61) (end 79.22 109.3353) (width 0.25) (layer F.Cu) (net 14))
 (segment (start 144.88 105.41) (end 142.9547 105.41) (width 0.25) (layer F.Cu) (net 14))
 (segment (start 82.55 58.9753) (end 79.22 62.3053) (width 0.25) (layer F.Cu) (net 14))
 (segment (start 79.22 62.3053) (end 79.22 107.61) (width 0.25) (layer F.Cu) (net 14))
 (segment (start 82.55 57.25) (end 82.55 58.9753) (width 0.25) (layer F.Cu) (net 14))
 (segment (start 74.14 107.61) (end 74.14 105.6847) (width 0.25) (layer F.Cu) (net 15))
 (segment (start 74.14 105.6847) (end 63.98 105.6847) (width 0.25) (layer F.Cu) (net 15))
 (segment (start 62.46 92.2) (end 62.46 93.4253) (width 0.25) (layer F.Cu) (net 15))
 (segment (start 63.98 107.61) (end 63.98 105.6847) (width 0.25) (layer F.Cu) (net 15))
 (segment (start 63.98 105.6847) (end 63.7946 105.4993) (width 0.25) (layer F.Cu) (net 15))
 (segment (start 63.7946 105.4993) (end 63.7946 94.7599) (width 0.25) (layer F.Cu) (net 15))
 (segment (start 63.7946 94.7599) (end 62.46 93.4253) (width 0.25) (layer F.Cu) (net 15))
 (segment (start 74.14 108.4726) (end 75.453 109.7856) (width 0.25) (layer B.Cu) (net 15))
 (segment (start 75.453 109.7856) (end 101.6297 109.7856) (width 0.25) (layer B.Cu) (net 15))
 (segment (start 101.6297 109.7856) (end 102.08 109.3353) (width 0.25) (layer B.Cu) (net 15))
 (segment (start 99.48 94.0547) (end 118.1059 94.0547) (width 0.25) (layer B.Cu) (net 15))
 (segment (start 118.1059 94.0547) (end 119.2447 95.1935) (width 0.25) (layer B.Cu) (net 15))
 (segment (start 120.47 92.8682) (end 130.81 82.5282) (width 0.25) (layer F.Cu) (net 15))
 (segment (start 130.81 82.5282) (end 130.81 62.33) (width 0.25) (layer F.Cu) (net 15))
 (segment (start 120.47 95.1935) (end 120.47 92.8682) (width 0.25) (layer F.Cu) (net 15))
 (segment (start 102.08 107.41) (end 102.08 109.3353) (width 0.25) (layer B.Cu) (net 15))
 (segment (start 74.14 107.61) (end 74.14 108.4726) (width 0.25) (layer B.Cu) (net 15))
 (segment (start 120.47 95.1935) (end 119.2447 95.1935) (width 0.25) (layer B.Cu) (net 15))
 (segment (start 99.48 95.28) (end 99.48 94.0547) (width 0.25) (layer B.Cu) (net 15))
 (segment (start 99.48 95.28) (end 99.48 96.5053) (width 0.25) (layer F.Cu) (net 15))
 (segment (start 102.08 107.41) (end 102.08 99.1053) (width 0.25) (layer F.Cu) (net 15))
 (segment (start 102.08 99.1053) (end 99.48 96.5053) (width 0.25) (layer F.Cu) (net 15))
 (segment (start 130.81 57.25) (end 130.81 62.33) (width 1) (layer F.Cu) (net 15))
 (segment (start 124.2447 95.1935) (end 115.1044 104.3338) (width 0.25) (layer B.Cu) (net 17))
 (segment (start 115.1044 104.3338) (end 72.9509 104.3338) (width 0.25) (layer B.Cu) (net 17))
 (segment (start 72.9509 104.3338) (end 71.6 105.6847) (width 0.25) (layer B.Cu) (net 17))
 (segment (start 120.41 89.96) (end 122.2353 89.96) (width 0.25) (layer B.Cu) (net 17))
 (segment (start 125.4317 95.1935) (end 124.2447 95.1935) (width 0.25) (layer B.Cu) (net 17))
 (segment (start 125.47 95.1935) (end 125.4317 95.1935) (width 0.25) (layer B.Cu) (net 17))
 (segment (start 122.2353 89.96) (end 125.4317 93.1564) (width 0.25) (layer B.Cu) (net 17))
 (segment (start 125.4317 93.1564) (end 125.4317 95.1935) (width 0.25) (layer B.Cu) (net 17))
 (segment (start 71.6 107.41) (end 71.6 105.6847) (width 0.25) (layer B.Cu) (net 17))
 (segment (start 69.06 107.61) (end 69.06 105.6847) (width 0.25) (layer B.Cu) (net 18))
 (segment (start 69.06 105.6847) (end 78.2394 96.5053) (width 0.25) (layer B.Cu) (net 18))
 (segment (start 78.2394 96.5053) (end 87.86 96.5053) (width 0.25) (layer B.Cu) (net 18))
 (segment (start 87.86 95.28) (end 87.86 96.5053) (width 0.25) (layer B.Cu) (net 18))
 (segment (start 107.1 95.28) (end 107.1 96.5053) (width 0.25) (layer B.Cu) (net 18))
 (segment (start 107.1 96.5053) (end 87.86 96.5053) (width 0.25) (layer B.Cu) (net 18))
 (segment (start 99.54 107.61) (end 99.54 109.3353) (width 0.25) (layer F.Cu) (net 19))
 (segment (start 99.54 109.3353) (end 102.5944 109.3353) (width 0.25) (layer F.Cu) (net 19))
 (segment (start 102.5944 109.3353) (end 115.57 96.3597) (width 0.25) (layer F.Cu) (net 19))
 (segment (start 115.57 96.3597) (end 115.57 57.15) (width 0.25) (layer F.Cu) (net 19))
 (segment (start 67.52 97.4335) (end 68.7453 97.4335) (width 0.25) (layer F.Cu) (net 1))
 (segment (start 68.7453 97.4335) (end 72.2329 93.9459) (width 0.25) (layer F.Cu) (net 1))
 (segment (start 72.2329 93.9459) (end 73.4458 93.9459) (width 0.25) (layer F.Cu) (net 1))
 (segment (start 62.52 97.4335) (end 62.52 95.1082) (width 0.25) (layer B.Cu) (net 16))
 (segment (start 70.08 92.2) (end 65.4282 92.2) (width 0.25) (layer B.Cu) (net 16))
 (segment (start 65.4282 92.2) (end 62.52 95.1082) (width 0.25) (layer B.Cu) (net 16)))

